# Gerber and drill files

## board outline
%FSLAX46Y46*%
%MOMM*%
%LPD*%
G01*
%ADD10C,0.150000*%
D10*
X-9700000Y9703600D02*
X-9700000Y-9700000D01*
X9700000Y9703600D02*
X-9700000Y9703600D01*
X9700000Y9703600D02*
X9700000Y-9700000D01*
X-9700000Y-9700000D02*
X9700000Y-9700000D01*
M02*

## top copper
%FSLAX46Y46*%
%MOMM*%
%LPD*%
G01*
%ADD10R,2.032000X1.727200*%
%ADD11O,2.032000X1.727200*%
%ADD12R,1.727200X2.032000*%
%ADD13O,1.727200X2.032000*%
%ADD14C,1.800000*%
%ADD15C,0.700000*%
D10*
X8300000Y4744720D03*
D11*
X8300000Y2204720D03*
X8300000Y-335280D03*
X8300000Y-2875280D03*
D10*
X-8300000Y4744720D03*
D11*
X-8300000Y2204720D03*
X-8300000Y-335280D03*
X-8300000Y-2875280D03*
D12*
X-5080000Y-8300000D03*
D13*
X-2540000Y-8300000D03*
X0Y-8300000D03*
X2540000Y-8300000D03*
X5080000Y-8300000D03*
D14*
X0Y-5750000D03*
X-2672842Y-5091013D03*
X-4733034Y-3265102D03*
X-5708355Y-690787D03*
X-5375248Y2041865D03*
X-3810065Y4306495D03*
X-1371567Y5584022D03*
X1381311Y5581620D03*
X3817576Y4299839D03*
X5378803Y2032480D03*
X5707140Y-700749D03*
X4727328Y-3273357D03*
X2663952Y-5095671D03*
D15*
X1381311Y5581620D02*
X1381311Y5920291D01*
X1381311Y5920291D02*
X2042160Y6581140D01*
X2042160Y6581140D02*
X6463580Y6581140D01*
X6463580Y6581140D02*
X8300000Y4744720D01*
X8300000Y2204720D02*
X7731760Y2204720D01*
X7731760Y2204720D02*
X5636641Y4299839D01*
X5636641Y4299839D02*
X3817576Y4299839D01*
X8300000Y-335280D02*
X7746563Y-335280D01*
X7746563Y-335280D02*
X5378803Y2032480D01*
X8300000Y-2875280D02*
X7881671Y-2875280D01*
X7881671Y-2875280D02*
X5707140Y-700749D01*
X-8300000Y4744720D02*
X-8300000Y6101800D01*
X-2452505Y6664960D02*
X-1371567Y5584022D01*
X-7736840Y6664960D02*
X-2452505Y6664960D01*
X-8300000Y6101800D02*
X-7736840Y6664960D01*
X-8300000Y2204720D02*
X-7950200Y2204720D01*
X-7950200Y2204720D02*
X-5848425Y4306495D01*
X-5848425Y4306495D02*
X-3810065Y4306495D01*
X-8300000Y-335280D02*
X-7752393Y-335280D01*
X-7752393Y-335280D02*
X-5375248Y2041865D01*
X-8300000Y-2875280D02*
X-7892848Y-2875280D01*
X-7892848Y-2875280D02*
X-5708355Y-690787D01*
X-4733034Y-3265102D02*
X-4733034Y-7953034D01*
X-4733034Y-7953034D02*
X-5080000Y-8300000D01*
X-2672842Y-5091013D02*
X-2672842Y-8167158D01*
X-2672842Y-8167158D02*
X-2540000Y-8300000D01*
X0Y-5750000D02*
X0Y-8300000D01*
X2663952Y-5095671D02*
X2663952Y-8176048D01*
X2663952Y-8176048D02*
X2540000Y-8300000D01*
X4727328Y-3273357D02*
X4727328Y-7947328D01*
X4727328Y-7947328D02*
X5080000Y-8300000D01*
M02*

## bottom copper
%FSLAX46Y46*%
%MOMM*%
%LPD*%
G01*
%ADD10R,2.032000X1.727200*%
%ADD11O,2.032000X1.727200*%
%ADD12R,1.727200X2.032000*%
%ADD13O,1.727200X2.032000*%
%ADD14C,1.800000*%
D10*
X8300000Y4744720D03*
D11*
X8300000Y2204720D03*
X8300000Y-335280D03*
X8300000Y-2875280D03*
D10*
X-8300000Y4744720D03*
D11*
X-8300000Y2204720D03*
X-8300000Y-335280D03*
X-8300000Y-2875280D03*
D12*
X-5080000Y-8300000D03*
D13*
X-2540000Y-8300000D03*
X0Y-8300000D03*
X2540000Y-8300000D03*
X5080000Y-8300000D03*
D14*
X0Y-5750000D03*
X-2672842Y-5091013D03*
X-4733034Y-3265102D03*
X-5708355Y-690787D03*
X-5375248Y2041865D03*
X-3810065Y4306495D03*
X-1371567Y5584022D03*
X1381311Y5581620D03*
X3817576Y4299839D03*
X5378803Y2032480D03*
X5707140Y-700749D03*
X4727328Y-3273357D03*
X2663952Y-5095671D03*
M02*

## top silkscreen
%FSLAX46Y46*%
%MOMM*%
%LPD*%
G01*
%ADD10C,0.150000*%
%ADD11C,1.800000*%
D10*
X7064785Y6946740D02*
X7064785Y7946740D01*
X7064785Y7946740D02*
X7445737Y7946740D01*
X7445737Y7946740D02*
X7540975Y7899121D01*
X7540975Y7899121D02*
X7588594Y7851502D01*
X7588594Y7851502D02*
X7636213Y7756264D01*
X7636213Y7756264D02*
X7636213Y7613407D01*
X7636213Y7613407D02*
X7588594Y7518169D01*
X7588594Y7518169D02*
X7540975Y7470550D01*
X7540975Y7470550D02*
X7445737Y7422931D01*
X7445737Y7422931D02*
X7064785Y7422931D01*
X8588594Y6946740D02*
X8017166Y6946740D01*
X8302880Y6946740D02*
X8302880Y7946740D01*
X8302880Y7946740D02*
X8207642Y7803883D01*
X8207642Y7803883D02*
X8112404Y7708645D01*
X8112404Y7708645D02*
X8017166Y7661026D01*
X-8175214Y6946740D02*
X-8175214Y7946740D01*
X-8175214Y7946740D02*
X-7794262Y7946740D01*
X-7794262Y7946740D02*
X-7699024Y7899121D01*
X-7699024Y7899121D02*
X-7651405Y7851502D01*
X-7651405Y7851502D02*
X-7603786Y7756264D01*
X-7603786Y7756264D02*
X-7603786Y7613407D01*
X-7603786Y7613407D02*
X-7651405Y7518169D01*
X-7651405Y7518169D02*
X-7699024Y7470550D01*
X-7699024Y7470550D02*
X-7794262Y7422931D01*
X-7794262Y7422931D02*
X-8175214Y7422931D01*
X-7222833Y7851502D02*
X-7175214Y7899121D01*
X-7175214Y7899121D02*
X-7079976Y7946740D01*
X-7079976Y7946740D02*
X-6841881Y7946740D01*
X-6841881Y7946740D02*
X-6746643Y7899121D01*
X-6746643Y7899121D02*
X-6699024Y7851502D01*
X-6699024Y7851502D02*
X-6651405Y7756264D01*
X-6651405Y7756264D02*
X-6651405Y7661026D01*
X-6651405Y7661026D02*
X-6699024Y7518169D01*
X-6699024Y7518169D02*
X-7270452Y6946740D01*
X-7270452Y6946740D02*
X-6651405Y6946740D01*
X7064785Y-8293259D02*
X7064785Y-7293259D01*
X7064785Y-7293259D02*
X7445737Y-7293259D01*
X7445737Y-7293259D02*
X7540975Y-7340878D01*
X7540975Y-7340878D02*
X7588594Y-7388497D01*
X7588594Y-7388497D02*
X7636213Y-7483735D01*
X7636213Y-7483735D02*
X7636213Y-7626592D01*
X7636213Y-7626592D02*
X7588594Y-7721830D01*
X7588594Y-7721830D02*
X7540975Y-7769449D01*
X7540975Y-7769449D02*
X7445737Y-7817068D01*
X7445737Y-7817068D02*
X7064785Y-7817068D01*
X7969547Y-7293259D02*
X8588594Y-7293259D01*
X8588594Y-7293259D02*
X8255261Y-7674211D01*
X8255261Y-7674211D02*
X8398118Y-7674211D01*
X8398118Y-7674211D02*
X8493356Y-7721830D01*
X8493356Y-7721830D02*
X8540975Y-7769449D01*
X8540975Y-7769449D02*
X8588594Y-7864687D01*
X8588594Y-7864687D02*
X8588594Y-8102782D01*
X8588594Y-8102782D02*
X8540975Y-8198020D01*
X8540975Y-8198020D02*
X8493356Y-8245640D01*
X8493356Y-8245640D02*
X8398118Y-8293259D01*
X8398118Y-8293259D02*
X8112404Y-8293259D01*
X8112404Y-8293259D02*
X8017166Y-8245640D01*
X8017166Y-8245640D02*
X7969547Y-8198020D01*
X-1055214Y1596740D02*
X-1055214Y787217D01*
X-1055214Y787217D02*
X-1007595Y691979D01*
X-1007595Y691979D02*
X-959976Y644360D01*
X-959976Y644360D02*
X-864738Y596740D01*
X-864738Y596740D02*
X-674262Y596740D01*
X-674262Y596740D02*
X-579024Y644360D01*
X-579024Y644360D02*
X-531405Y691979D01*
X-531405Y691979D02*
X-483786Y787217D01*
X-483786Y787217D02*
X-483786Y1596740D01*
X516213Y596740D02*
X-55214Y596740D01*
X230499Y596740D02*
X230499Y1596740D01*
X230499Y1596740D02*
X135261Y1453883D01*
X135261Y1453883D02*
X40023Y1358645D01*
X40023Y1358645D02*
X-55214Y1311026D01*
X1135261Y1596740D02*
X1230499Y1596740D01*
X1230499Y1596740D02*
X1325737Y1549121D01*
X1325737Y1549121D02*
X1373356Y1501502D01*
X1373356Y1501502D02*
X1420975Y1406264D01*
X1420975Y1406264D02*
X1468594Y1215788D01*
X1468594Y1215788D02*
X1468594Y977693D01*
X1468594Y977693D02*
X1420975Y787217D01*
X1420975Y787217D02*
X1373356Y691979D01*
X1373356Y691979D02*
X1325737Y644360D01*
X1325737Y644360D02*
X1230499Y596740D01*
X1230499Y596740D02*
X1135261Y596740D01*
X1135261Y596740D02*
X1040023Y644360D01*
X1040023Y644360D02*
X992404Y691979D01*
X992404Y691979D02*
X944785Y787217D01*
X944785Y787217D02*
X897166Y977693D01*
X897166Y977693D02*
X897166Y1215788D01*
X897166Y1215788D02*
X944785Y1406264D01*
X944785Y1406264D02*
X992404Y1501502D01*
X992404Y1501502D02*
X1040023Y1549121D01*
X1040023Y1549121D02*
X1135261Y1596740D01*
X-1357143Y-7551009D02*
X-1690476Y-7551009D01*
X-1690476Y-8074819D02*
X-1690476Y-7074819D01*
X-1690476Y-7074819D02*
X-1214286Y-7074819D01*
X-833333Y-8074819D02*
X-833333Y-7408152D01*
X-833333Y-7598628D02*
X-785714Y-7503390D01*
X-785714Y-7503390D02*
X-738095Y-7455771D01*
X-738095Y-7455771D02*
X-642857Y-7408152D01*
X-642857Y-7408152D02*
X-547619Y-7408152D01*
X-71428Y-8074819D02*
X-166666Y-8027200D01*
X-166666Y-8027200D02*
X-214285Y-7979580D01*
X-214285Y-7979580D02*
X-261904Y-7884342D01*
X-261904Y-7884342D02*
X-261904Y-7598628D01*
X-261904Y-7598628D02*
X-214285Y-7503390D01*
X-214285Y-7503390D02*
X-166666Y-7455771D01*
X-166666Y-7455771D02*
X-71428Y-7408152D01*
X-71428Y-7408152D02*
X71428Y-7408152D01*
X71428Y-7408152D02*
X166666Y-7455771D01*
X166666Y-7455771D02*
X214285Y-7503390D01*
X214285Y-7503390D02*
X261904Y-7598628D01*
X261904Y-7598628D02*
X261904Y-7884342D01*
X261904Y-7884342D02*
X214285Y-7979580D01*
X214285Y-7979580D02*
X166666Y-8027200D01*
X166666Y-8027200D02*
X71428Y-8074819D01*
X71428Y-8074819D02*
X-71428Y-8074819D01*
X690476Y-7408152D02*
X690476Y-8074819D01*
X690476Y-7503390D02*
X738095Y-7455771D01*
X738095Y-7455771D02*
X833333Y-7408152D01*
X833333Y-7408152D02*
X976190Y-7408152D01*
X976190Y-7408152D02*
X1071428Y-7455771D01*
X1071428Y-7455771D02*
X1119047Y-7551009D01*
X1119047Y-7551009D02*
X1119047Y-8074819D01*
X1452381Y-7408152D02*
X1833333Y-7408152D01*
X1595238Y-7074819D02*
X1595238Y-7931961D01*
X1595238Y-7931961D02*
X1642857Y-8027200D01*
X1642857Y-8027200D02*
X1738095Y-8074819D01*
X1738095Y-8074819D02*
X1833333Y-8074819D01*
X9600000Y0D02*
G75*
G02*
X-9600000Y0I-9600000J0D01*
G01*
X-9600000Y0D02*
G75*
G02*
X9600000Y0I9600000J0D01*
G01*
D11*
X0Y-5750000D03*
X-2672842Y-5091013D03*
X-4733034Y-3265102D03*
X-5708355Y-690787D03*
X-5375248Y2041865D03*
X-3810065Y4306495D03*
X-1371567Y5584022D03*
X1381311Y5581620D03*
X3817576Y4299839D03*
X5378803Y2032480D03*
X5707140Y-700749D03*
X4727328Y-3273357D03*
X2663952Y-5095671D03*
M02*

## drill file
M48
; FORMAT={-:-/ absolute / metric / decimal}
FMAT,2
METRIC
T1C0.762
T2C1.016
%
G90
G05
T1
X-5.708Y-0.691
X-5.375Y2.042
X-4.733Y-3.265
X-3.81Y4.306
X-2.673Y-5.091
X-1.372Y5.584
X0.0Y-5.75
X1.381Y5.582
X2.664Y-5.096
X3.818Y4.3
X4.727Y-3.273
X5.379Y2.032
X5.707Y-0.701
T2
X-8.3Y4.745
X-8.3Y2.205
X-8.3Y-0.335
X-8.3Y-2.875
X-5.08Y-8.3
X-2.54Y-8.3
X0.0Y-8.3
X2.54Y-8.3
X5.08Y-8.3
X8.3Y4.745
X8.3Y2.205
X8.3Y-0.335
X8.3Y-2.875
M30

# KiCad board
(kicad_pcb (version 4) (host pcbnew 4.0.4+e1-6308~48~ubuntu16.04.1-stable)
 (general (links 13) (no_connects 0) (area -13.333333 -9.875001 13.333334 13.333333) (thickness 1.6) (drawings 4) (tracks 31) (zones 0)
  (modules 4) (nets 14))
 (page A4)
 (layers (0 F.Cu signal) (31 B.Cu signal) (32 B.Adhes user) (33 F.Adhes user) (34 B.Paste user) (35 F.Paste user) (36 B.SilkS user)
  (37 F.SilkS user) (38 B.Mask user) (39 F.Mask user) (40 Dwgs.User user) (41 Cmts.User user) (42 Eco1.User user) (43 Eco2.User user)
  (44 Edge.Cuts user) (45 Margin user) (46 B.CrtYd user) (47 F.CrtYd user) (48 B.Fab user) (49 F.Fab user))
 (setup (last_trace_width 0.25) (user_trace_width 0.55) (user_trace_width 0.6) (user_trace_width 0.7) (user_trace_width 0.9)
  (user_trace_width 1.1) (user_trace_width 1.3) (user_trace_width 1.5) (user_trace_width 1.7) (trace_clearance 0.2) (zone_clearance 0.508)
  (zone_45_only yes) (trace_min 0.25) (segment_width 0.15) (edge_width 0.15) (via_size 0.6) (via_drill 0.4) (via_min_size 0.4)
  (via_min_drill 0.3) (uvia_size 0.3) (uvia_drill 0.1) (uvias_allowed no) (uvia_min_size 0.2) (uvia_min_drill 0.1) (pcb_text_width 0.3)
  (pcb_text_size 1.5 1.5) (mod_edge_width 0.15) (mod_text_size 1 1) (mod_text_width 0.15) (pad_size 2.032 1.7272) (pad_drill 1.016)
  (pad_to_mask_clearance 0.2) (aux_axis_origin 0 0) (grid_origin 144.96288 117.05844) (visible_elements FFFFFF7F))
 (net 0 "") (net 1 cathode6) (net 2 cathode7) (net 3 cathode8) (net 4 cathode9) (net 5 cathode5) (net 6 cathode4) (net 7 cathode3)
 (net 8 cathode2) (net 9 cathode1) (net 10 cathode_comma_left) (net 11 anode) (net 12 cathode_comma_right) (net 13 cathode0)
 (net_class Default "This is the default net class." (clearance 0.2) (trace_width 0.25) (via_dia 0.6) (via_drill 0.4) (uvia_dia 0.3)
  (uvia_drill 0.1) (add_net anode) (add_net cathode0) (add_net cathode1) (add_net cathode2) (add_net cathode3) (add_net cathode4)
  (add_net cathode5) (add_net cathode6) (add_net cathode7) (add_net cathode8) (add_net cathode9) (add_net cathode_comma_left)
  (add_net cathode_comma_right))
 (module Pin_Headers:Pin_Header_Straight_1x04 (layer B.Cu) (at 8.3 -4.74472 180)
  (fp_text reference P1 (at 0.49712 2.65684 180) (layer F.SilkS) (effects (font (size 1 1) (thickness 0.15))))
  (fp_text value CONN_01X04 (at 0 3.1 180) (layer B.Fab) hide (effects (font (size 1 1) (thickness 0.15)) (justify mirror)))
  (pad 1 thru_hole rect (at 0 0 180) (size 2.032 1.7272) (drill 1.016) (layers *.Cu *.Mask B.SilkS) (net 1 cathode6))
  (pad 2 thru_hole oval (at 0 -2.54 180) (size 2.032 1.7272) (drill 1.016) (layers *.Cu *.Mask B.SilkS) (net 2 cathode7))
  (pad 3 thru_hole oval (at 0 -5.08 180) (size 2.032 1.7272) (drill 1.016) (layers *.Cu *.Mask B.SilkS) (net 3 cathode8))
  (pad 4 thru_hole oval (at 0 -7.62 180) (size 2.032 1.7272) (drill 1.016) (layers *.Cu *.Mask B.SilkS) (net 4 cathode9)))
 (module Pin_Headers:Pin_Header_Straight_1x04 (layer B.Cu) (at -8.3 -4.74472 180)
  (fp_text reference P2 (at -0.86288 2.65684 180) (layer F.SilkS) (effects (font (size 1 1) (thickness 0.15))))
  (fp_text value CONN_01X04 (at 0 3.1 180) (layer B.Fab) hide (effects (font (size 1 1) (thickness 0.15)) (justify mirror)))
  (pad 1 thru_hole rect (at 0 0 180) (size 2.032 1.7272) (drill 1.016) (layers *.Cu *.Mask B.SilkS) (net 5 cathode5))
  (pad 2 thru_hole oval (at 0 -2.54 180) (size 2.032 1.7272) (drill 1.016) (layers *.Cu *.Mask B.SilkS) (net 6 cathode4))
  (pad 3 thru_hole oval (at 0 -5.08 180) (size 2.032 1.7272) (drill 1.016) (layers *.Cu *.Mask B.SilkS) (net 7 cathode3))
  (pad 4 thru_hole oval (at 0 -7.62 180) (size 2.032 1.7272) (drill 1.016) (layers *.Cu *.Mask B.SilkS) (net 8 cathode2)))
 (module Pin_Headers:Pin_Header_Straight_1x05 (layer B.Cu) (at -5.08 8.3 270)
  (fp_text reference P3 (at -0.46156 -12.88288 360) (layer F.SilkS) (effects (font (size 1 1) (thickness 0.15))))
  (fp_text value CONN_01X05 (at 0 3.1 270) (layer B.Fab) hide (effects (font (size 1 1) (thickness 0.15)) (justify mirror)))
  (pad 1 thru_hole rect (at 0 0 270) (size 2.032 1.7272) (drill 1.016) (layers *.Cu *.Mask B.SilkS) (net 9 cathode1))
  (pad 2 thru_hole oval (at 0 -2.54 270) (size 2.032 1.7272) (drill 1.016) (layers *.Cu *.Mask B.SilkS) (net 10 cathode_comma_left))
  (pad 3 thru_hole oval (at 0 -5.08 270) (size 2.032 1.7272) (drill 1.016) (layers *.Cu *.Mask B.SilkS) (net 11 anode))
  (pad 4 thru_hole oval (at 0 -7.62 270) (size 2.032 1.7272) (drill 1.016) (layers *.Cu *.Mask B.SilkS) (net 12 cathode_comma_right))
  (pad 5 thru_hole oval (at 0 -10.16 270) (size 2.032 1.7272) (drill 1.016) (layers *.Cu *.Mask B.SilkS) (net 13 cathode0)))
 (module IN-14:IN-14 (layer F.Cu) (at 0 0)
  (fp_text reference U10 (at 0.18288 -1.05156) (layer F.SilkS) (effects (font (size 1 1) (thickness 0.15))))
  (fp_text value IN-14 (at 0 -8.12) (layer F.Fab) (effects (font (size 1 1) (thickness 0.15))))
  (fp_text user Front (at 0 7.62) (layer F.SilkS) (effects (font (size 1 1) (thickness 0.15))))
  (fp_circle (center 0 0) (end 0 9.6) (layer F.SilkS) (width 0.15))
  (pad 1 thru_hole circle (at 0 5.75) (size 1.8 1.8) (drill 0.762) (layers *.Cu *.Mask F.SilkS) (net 11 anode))
  (pad 2 thru_hole circle (at -2.672842 5.091013) (size 1.8 1.8) (drill 0.762) (layers *.Cu *.Mask F.SilkS) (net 10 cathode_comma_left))
  (pad 3 thru_hole circle (at -4.733034 3.265102) (size 1.8 1.8) (drill 0.762) (layers *.Cu *.Mask F.SilkS) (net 9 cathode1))
  (pad 4 thru_hole circle (at -5.708355 0.690787) (size 1.8 1.8) (drill 0.762) (layers *.Cu *.Mask F.SilkS) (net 8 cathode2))
  (pad 5 thru_hole circle (at -5.375248 -2.041865) (size 1.8 1.8) (drill 0.762) (layers *.Cu *.Mask F.SilkS) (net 7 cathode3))
  (pad 6 thru_hole circle (at -3.810065 -4.306495) (size 1.8 1.8) (drill 0.762) (layers *.Cu *.Mask F.SilkS) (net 6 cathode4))
  (pad 7 thru_hole circle (at -1.371567 -5.584022) (size 1.8 1.8) (drill 0.762) (layers *.Cu *.Mask F.SilkS) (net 5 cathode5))
  (pad 8 thru_hole circle (at 1.381311 -5.58162) (size 1.8 1.8) (drill 0.762) (layers *.Cu *.Mask F.SilkS) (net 1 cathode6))
  (pad 9 thru_hole circle (at 3.817576 -4.299839) (size 1.8 1.8) (drill 0.762) (layers *.Cu *.Mask F.SilkS) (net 2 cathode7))
  (pad 10 thru_hole circle (at 5.378803 -2.03248) (size 1.8 1.8) (drill 0.762) (layers *.Cu *.Mask F.SilkS) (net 3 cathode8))
  (pad 11 thru_hole circle (at 5.70714 0.700749) (size 1.8 1.8) (drill 0.762) (layers *.Cu *.Mask F.SilkS) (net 4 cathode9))
  (pad 12 thru_hole circle (at 4.727328 3.273357) (size 1.8 1.8) (drill 0.762) (layers *.Cu *.Mask F.SilkS) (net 13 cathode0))
  (pad 13 thru_hole circle (at 2.663952 5.095671) (size 1.8 1.8) (drill 0.762) (layers *.Cu *.Mask F.SilkS) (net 12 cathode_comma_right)))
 (gr_line (start -9.7 -9.7036) (end -9.7 9.7) (angle 90) (layer Edge.Cuts) (width 0.15))
 (gr_line (start 9.7 -9.7036) (end -9.7 -9.7036) (angle 90) (layer Edge.Cuts) (width 0.15))
 (gr_line (start 9.7 -9.7036) (end 9.7 9.7) (angle 90) (layer Edge.Cuts) (width 0.15))
 (gr_line (start -9.7 9.7) (end 9.7 9.7) (angle 90) (layer Edge.Cuts) (width 0.15))
 (segment (start 1.381311 -5.58162) (end 1.381311 -5.920291) (width 0.7) (layer F.Cu) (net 1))
 (segment (start 1.381311 -5.920291) (end 2.04216 -6.58114) (width 0.7) (layer F.Cu) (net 1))
 (segment (start 2.04216 -6.58114) (end 6.46358 -6.58114) (width 0.7) (layer F.Cu) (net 1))
 (segment (start 6.46358 -6.58114) (end 8.3 -4.74472) (width 0.7) (layer F.Cu) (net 1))
 (segment (start 8.3 -2.20472) (end 7.73176 -2.20472) (width 0.7) (layer F.Cu) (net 2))
 (segment (start 7.73176 -2.20472) (end 5.636641 -4.299839) (width 0.7) (layer F.Cu) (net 2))
 (segment (start 5.636641 -4.299839) (end 3.817576 -4.299839) (width 0.7) (layer F.Cu) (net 2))
 (segment (start 8.3 0.33528) (end 7.746563 0.33528) (width 0.7) (layer F.Cu) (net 3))
 (segment (start 7.746563 0.33528) (end 5.378803 -2.03248) (width 0.7) (layer F.Cu) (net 3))
 (segment (start 8.3 2.87528) (end 7.881671 2.87528) (width 0.7) (layer F.Cu) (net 4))
 (segment (start 7.881671 2.87528) (end 5.70714 0.700749) (width 0.7) (layer F.Cu) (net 4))
 (segment (start -8.3 -4.74472) (end -8.3 -6.1018) (width 0.7) (layer F.Cu) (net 5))
 (segment (start -2.452505 -6.66496) (end -1.371567 -5.584022) (width 0.7) (layer F.Cu) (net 5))
 (segment (start -7.73684 -6.66496) (end -2.452505 -6.66496) (width 0.7) (layer F.Cu) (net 5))
 (segment (start -8.3 -6.1018) (end -7.73684 -6.66496) (width 0.7) (layer F.Cu) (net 5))
 (segment (start -8.3 -2.20472) (end -7.9502 -2.20472) (width 0.7) (layer F.Cu) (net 6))
 (segment (start -7.9502 -2.20472) (end -5.848425 -4.306495) (width 0.7) (layer F.Cu) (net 6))
 (segment (start -5.848425 -4.306495) (end -3.810065 -4.306495) (width 0.7) (layer F.Cu) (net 6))
 (segment (start -8.3 0.33528) (end -7.752393 0.33528) (width 0.7) (layer F.Cu) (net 7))
 (segment (start -7.752393 0.33528) (end -5.375248 -2.041865) (width 0.7) (layer F.Cu) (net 7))
 (segment (start -8.3 2.87528) (end -7.892848 2.87528) (width 0.7) (layer F.Cu) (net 8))
 (segment (start -7.892848 2.87528) (end -5.708355 0.690787) (width 0.7) (layer F.Cu) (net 8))
 (segment (start -4.733034 3.265102) (end -4.733034 7.953034) (width 0.7) (layer F.Cu) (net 9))
 (segment (start -4.733034 7.953034) (end -5.08 8.3) (width 0.7) (layer F.Cu) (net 9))
 (segment (start -2.672842 5.091013) (end -2.672842 8.167158) (width 0.7) (layer F.Cu) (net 10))
 (segment (start -2.672842 8.167158) (end -2.54 8.3) (width 0.7) (layer F.Cu) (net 10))
 (segment (start 0 5.75) (end 0 8.3) (width 0.7) (layer F.Cu) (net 11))
 (segment (start 2.663952 5.095671) (end 2.663952 8.176048) (width 0.7) (layer F.Cu) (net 12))
 (segment (start 2.663952 8.176048) (end 2.54 8.3) (width 0.7) (layer F.Cu) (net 12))
 (segment (start 4.727328 3.273357) (end 4.727328 7.947328) (width 0.7) (layer F.Cu) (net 13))
 (segment (start 4.727328 7.947328) (end 5.08 8.3) (width 0.7) (layer F.Cu) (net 13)))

